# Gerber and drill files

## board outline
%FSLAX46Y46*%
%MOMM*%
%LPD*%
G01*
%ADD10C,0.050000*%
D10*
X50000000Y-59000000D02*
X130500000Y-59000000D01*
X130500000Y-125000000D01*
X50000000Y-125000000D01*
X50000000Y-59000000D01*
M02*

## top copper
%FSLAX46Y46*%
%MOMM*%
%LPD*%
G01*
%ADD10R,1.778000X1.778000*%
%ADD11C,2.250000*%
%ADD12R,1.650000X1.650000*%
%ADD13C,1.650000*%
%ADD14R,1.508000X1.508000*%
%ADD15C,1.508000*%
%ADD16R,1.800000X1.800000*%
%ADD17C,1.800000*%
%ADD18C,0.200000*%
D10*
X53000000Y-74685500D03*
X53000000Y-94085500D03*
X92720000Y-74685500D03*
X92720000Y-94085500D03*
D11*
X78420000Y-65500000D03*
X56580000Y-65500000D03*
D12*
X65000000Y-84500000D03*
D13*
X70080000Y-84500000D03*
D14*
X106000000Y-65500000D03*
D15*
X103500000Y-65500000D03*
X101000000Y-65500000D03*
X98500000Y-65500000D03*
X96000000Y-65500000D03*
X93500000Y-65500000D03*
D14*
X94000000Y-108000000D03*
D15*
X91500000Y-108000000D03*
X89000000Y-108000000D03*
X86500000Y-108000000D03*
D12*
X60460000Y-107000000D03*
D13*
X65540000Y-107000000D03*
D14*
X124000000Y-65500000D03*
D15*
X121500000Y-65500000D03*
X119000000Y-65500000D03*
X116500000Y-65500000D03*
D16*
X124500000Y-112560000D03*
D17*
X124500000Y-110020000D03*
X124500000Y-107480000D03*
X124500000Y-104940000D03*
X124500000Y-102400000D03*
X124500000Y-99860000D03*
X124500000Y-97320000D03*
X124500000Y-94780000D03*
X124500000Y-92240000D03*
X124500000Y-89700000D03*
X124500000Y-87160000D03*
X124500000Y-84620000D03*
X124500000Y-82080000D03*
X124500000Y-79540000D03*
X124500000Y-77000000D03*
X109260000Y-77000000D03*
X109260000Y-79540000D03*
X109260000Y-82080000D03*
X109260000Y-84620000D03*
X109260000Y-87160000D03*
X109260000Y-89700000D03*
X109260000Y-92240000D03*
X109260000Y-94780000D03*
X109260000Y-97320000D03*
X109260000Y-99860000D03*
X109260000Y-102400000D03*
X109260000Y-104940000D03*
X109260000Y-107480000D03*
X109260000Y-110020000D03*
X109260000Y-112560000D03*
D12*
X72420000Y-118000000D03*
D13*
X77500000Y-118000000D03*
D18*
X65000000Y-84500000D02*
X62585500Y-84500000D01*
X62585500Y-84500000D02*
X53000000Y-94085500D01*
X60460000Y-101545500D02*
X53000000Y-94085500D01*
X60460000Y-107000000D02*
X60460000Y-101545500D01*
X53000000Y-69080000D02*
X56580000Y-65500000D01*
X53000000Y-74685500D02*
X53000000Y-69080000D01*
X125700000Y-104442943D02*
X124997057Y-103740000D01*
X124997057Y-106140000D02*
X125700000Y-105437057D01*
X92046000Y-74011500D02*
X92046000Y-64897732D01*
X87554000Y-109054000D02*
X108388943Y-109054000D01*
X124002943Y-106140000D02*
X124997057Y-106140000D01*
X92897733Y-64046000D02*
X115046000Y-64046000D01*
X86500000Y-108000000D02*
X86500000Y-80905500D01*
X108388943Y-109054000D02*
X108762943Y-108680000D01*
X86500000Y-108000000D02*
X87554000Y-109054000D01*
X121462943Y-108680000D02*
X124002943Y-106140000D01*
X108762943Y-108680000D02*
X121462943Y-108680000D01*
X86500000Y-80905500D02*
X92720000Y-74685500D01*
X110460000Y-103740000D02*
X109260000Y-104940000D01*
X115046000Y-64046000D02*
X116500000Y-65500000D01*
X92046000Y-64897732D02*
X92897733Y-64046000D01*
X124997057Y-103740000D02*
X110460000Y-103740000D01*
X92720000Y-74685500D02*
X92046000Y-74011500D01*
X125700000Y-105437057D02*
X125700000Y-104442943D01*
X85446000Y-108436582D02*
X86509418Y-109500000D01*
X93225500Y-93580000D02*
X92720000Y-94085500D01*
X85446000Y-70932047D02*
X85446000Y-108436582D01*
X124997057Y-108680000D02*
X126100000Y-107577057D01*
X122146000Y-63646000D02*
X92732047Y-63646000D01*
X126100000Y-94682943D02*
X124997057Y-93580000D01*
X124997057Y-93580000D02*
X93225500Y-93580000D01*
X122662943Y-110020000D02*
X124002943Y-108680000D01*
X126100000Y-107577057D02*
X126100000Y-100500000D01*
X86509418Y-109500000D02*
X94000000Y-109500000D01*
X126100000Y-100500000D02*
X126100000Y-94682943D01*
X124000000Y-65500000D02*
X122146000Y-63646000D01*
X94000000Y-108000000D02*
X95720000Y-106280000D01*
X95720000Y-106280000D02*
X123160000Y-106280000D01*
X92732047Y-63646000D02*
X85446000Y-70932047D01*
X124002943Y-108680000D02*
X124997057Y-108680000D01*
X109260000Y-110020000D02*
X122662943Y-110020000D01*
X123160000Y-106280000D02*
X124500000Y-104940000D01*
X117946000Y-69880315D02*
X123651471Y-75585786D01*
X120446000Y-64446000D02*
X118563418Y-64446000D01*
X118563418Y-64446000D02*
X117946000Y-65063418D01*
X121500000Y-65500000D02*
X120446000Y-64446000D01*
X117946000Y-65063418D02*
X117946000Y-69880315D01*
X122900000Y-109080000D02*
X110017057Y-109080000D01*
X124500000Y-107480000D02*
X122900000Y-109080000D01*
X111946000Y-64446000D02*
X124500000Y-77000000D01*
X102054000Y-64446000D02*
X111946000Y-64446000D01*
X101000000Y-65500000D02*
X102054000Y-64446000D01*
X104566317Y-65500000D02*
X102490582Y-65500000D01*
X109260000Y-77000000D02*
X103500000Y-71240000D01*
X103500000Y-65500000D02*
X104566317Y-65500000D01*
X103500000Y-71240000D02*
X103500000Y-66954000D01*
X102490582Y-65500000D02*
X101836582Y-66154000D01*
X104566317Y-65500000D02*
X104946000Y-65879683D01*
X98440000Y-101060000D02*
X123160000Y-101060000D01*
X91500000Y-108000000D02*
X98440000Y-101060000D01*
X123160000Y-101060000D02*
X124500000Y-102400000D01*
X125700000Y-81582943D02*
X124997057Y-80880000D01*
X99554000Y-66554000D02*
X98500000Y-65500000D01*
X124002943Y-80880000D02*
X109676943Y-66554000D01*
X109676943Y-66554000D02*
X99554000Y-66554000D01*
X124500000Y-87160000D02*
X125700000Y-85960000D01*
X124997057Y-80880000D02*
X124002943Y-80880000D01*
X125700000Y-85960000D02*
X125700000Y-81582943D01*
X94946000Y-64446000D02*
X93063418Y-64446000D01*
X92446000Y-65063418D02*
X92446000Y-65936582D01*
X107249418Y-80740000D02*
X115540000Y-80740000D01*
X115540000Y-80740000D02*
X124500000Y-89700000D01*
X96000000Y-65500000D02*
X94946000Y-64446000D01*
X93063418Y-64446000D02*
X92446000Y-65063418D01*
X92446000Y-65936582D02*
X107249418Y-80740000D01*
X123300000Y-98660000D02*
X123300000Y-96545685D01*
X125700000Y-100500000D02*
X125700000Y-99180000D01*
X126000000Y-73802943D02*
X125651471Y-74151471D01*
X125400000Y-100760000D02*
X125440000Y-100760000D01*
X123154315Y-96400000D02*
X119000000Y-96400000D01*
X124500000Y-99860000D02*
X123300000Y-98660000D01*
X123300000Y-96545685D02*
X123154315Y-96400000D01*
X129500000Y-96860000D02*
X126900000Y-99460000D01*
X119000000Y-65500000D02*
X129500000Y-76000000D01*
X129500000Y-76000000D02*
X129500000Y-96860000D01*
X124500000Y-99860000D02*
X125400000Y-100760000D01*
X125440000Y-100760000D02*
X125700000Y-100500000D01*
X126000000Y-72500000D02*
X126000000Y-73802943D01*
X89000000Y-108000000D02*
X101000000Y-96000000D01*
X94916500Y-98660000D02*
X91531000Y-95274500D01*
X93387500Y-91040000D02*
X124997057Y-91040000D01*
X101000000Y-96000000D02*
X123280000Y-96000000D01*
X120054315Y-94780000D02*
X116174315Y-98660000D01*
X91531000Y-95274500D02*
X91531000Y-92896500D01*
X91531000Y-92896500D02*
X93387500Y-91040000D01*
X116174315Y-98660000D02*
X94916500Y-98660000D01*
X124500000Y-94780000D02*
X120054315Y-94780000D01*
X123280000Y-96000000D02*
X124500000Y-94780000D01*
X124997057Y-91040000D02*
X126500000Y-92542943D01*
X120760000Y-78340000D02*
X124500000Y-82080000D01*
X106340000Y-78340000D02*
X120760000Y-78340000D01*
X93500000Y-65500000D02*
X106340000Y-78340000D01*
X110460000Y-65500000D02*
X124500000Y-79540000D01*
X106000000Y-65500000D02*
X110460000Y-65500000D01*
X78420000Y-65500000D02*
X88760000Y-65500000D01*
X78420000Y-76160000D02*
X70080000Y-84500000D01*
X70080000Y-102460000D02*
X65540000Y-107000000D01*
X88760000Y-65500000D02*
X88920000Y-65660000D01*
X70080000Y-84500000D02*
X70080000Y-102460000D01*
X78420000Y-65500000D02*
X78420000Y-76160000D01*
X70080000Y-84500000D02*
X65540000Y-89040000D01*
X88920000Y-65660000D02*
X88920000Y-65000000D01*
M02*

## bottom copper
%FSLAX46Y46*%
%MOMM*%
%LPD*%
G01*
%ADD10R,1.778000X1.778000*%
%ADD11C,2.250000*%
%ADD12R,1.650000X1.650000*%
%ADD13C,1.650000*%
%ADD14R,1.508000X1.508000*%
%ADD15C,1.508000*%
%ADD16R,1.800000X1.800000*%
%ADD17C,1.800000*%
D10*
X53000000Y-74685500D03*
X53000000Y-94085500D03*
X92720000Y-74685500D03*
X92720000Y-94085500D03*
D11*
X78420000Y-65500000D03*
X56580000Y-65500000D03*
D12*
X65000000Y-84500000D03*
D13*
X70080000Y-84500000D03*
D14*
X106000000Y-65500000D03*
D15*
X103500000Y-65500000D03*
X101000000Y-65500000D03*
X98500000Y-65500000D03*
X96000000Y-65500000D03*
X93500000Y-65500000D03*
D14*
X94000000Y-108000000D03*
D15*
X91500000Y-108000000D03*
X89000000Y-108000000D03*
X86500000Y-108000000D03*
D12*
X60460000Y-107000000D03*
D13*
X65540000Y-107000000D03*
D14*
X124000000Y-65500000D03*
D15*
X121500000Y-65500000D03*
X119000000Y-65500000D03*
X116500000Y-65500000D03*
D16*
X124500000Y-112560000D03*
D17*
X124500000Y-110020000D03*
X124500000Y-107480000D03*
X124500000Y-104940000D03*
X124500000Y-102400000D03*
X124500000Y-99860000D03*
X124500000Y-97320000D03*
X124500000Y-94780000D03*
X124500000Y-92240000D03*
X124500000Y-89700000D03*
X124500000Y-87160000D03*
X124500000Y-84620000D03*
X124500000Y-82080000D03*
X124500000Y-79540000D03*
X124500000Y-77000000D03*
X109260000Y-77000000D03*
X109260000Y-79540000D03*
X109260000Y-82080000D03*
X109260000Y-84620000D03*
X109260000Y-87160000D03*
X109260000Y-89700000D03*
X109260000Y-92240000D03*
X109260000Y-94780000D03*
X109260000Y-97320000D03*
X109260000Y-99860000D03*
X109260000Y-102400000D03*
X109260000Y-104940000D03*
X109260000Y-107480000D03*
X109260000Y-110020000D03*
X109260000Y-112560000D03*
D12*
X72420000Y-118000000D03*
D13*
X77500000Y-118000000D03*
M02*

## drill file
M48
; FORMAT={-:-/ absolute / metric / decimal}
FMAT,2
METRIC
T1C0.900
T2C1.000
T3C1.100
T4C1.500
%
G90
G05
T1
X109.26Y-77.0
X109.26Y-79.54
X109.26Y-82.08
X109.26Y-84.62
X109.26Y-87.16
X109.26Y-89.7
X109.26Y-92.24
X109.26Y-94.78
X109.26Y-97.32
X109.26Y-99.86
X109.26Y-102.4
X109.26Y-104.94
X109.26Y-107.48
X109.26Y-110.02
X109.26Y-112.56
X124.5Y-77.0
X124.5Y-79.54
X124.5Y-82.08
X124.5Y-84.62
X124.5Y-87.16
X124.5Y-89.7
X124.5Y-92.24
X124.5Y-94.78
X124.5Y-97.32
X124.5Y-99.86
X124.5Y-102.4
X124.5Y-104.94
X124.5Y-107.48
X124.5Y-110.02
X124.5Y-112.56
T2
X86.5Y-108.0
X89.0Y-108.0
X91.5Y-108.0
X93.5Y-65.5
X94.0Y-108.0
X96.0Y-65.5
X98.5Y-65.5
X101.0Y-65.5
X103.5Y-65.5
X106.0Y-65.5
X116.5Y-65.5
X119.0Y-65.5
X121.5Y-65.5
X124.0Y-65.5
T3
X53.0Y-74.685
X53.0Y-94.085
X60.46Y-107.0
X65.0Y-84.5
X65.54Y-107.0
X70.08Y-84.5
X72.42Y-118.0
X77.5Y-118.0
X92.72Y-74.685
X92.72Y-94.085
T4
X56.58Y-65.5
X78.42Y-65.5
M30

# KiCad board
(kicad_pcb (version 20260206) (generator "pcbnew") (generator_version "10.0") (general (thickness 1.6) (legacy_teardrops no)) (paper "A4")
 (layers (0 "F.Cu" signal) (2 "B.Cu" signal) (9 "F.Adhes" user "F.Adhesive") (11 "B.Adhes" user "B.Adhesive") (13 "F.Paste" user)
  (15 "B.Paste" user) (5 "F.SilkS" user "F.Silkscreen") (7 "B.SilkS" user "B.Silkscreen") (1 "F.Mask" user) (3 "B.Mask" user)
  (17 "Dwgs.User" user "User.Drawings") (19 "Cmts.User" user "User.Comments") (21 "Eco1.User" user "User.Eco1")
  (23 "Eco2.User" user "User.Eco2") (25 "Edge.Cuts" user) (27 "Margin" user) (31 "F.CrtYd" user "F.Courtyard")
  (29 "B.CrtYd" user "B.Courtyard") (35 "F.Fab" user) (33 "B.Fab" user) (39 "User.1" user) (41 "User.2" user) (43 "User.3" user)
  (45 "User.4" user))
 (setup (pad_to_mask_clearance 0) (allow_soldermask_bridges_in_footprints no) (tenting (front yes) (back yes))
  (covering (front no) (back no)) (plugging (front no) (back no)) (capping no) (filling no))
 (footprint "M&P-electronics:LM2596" (layer "F.Cu") (at 53 74.6855)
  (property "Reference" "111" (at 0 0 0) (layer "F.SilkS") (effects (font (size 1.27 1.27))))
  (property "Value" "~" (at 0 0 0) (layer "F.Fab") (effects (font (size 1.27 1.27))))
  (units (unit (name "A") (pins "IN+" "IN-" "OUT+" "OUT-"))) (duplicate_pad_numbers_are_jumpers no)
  (pad "IN+" thru_hole rect (at 0 0) (size 1.778 1.778) (drill 1.1) (layers "*.Cu" "*.Mask") (remove_unused_layers no)
   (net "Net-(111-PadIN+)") (solder_mask_margin 0.1016) (thermal_bridge_angle 0))
  (pad "IN-" thru_hole rect (at 0 19.4) (size 1.778 1.778) (drill 1.1) (layers "*.Cu" "*.Mask") (remove_unused_layers no)
   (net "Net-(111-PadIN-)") (solder_mask_margin 0.1016) (thermal_bridge_angle 0))
  (pad "OUT+" thru_hole rect (at 39.72 0) (size 1.778 1.778) (drill 1.1) (layers "*.Cu" "*.Mask") (remove_unused_layers no) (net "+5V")
   (solder_mask_margin 0.1016) (thermal_bridge_angle 0))
  (pad "OUT-" thru_hole rect (at 39.72 19.4) (size 1.778 1.778) (drill 1.1) (layers "*.Cu" "*.Mask") (remove_unused_layers no) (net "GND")
   (solder_mask_margin 0.1016) (thermal_bridge_angle 0)))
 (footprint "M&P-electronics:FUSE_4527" (layer "F.Cu") (at 67.5 65.5 180)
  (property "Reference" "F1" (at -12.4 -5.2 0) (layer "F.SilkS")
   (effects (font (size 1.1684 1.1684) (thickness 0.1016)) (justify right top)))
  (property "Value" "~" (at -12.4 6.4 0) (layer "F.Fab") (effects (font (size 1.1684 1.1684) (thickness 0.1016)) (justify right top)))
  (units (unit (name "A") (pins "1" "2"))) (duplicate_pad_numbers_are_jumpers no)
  (pad "1" thru_hole circle (at -10.92 0 180) (size 2.25 2.25) (drill 1.5) (layers "*.Cu" "*.Mask") (remove_unused_layers no)
   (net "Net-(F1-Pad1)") (solder_mask_margin 0.1016) (thermal_bridge_angle 0))
  (pad "2" thru_hole circle (at 10.92 0 180) (size 2.25 2.25) (drill 1.5) (layers "*.Cu" "*.Mask") (remove_unused_layers no)
   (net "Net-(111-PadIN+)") (solder_mask_margin 0.1016) (thermal_bridge_angle 0)))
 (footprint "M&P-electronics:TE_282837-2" (layer "F.Cu") (at 67.54 84.5)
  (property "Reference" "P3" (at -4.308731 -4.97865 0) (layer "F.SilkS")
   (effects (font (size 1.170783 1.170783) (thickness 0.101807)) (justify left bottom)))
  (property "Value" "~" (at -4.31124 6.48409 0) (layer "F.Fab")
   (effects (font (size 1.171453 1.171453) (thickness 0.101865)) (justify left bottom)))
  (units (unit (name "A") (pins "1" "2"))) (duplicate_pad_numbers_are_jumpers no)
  (pad "1" thru_hole rect (at -2.54 0) (size 1.65 1.65) (drill 1.1) (layers "*.Cu" "*.Mask") (remove_unused_layers no)
   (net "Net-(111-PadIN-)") (solder_mask_margin 0.1016) (thermal_bridge_angle 0))
  (pad "2" thru_hole circle (at 2.54 0) (size 1.65 1.65) (drill 1.1) (layers "*.Cu" "*.Mask") (remove_unused_layers no)
   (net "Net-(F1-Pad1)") (solder_mask_margin 0.1016) (thermal_bridge_angle 0)))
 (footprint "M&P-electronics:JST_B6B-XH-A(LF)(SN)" (layer "F.Cu") (at 99.75 64.975)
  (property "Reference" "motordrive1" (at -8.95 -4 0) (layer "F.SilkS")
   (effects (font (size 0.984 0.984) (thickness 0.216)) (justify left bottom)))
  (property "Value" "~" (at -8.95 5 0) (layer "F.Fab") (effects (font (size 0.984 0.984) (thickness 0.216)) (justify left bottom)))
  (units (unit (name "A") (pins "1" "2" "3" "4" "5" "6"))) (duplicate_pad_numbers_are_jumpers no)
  (pad "1" thru_hole rect (at 6.25 0.525) (size 1.508 1.508) (drill 1) (layers "*.Cu" "*.Mask") (remove_unused_layers no) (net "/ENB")
   (solder_mask_margin 0.1016) (thermal_bridge_angle 0))
  (pad "2" thru_hole circle (at 3.75 0.525) (size 1.508 1.508) (drill 1) (layers "*.Cu" "*.Mask") (remove_unused_layers no) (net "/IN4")
   (solder_mask_margin 0.1016) (thermal_bridge_angle 0))
  (pad "3" thru_hole circle (at 1.25 0.525) (size 1.508 1.508) (drill 1) (layers "*.Cu" "*.Mask") (remove_unused_layers no) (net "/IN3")
   (solder_mask_margin 0.1016) (thermal_bridge_angle 0))
  (pad "4" thru_hole circle (at -1.25 0.525) (size 1.508 1.508) (drill 1) (layers "*.Cu" "*.Mask") (remove_unused_layers no) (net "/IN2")
   (solder_mask_margin 0.1016) (thermal_bridge_angle 0))
  (pad "5" thru_hole circle (at -3.75 0.525) (size 1.508 1.508) (drill 1) (layers "*.Cu" "*.Mask") (remove_unused_layers no) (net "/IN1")
   (solder_mask_margin 0.1016) (thermal_bridge_angle 0))
  (pad "6" thru_hole circle (at -6.25 0.525) (size 1.508 1.508) (drill 1) (layers "*.Cu" "*.Mask") (remove_unused_layers no) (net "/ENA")
   (solder_mask_margin 0.1016) (thermal_bridge_angle 0)))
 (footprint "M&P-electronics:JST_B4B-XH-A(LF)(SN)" (layer "F.Cu") (at 90.25 107.475)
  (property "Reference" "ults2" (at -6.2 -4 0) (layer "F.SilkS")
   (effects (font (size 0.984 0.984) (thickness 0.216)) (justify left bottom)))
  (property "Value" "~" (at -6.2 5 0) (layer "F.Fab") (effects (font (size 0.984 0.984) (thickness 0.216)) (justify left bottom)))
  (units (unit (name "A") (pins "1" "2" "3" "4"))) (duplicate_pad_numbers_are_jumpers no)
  (pad "1" thru_hole rect (at 3.75 0.525) (size 1.508 1.508) (drill 1) (layers "*.Cu" "*.Mask") (remove_unused_layers no) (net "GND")
   (solder_mask_margin 0.1016) (thermal_bridge_angle 0))
  (pad "2" thru_hole circle (at 1.25 0.525) (size 1.508 1.508) (drill 1) (layers "*.Cu" "*.Mask") (remove_unused_layers no) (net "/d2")
   (solder_mask_margin 0.1016) (thermal_bridge_angle 0))
  (pad "3" thru_hole circle (at -1.25 0.525) (size 1.508 1.508) (drill 1) (layers "*.Cu" "*.Mask") (remove_unused_layers no) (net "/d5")
   (solder_mask_margin 0.1016) (thermal_bridge_angle 0))
  (pad "4" thru_hole circle (at -3.75 0.525) (size 1.508 1.508) (drill 1) (layers "*.Cu" "*.Mask") (remove_unused_layers no) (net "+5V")
   (solder_mask_margin 0.1016) (thermal_bridge_angle 0)))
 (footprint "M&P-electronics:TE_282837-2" (layer "F.Cu") (at 63 107)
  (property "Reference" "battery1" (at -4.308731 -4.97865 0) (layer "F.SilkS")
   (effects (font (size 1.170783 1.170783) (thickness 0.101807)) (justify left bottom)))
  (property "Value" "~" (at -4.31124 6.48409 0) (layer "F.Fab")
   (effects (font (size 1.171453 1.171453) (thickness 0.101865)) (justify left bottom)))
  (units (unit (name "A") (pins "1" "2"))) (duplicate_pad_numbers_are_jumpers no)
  (pad "1" thru_hole rect (at -2.54 0) (size 1.65 1.65) (drill 1.1) (layers "*.Cu" "*.Mask") (remove_unused_layers no)
   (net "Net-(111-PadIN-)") (solder_mask_margin 0.1016) (thermal_bridge_angle 0))
  (pad "2" thru_hole circle (at 2.54 0) (size 1.65 1.65) (drill 1.1) (layers "*.Cu" "*.Mask") (remove_unused_layers no)
   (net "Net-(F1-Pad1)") (solder_mask_margin 0.1016) (thermal_bridge_angle 0)))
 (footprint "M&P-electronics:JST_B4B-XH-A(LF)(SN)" (layer "F.Cu") (at 120.25 64.975)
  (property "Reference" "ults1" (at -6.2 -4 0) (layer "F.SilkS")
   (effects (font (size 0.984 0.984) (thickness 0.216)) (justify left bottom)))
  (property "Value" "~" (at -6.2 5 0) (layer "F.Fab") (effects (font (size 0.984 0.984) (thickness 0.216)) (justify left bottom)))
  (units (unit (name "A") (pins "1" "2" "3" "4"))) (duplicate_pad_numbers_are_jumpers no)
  (pad "1" thru_hole rect (at 3.75 0.525) (size 1.508 1.508) (drill 1) (layers "*.Cu" "*.Mask") (remove_unused_layers no) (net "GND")
   (solder_mask_margin 0.1016) (thermal_bridge_angle 0))
  (pad "2" thru_hole circle (at 1.25 0.525) (size 1.508 1.508) (drill 1) (layers "*.Cu" "*.Mask") (remove_unused_layers no) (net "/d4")
   (solder_mask_margin 0.1016) (thermal_bridge_angle 0))
  (pad "3" thru_hole circle (at -1.25 0.525) (size 1.508 1.508) (drill 1) (layers "*.Cu" "*.Mask") (remove_unused_layers no) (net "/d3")
   (solder_mask_margin 0.1016) (thermal_bridge_angle 0))
  (pad "4" thru_hole circle (at -3.75 0.525) (size 1.508 1.508) (drill 1) (layers "*.Cu" "*.Mask") (remove_unused_layers no) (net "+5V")
   (solder_mask_margin 0.1016) (thermal_bridge_angle 0)))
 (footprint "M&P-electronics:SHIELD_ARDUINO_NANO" (layer "F.Cu") (at 116.88 94.78 180)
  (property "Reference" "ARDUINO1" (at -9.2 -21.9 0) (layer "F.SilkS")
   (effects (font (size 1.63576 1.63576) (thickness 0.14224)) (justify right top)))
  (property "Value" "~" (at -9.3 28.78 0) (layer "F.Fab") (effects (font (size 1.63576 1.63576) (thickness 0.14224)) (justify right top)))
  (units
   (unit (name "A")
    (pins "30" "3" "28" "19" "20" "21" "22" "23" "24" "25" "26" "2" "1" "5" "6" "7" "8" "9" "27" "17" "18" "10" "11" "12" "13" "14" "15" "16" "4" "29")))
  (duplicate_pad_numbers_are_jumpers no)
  (pad "1" thru_hole rect (at -7.62 -17.78 90) (size 1.8 1.8) (drill 0.9) (layers "*.Cu" "*.Mask") (remove_unused_layers no)
   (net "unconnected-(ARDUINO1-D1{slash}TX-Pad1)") (solder_mask_margin 0.1016) (thermal_bridge_angle 0))
  (pad "2" thru_hole circle (at -7.62 -15.24 90) (size 1.8 1.8) (drill 0.9) (layers "*.Cu" "*.Mask") (remove_unused_layers no)
   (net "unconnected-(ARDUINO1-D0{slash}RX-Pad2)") (solder_mask_margin 0.1016) (thermal_bridge_angle 0))
  (pad "3" thru_hole circle (at -7.62 -12.7 90) (size 1.8 1.8) (drill 0.9) (layers "*.Cu" "*.Mask") (remove_unused_layers no)
   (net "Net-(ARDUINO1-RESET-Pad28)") (solder_mask_margin 0.1016) (thermal_bridge_angle 0))
  (pad "4" thru_hole circle (at -7.62 -10.16 90) (size 1.8 1.8) (drill 0.9) (layers "*.Cu" "*.Mask") (remove_unused_layers no) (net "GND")
   (solder_mask_margin 0.1016) (thermal_bridge_angle 0))
  (pad "5" thru_hole circle (at -7.62 -7.62 90) (size 1.8 1.8) (drill 0.9) (layers "*.Cu" "*.Mask") (remove_unused_layers no) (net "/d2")
   (solder_mask_margin 0.1016) (thermal_bridge_angle 0))
  (pad "6" thru_hole circle (at -7.62 -5.08 90) (size 1.8 1.8) (drill 0.9) (layers "*.Cu" "*.Mask") (remove_unused_layers no) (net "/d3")
   (solder_mask_margin 0.1016) (thermal_bridge_angle 0))
  (pad "7" thru_hole circle (at -7.62 -2.54 90) (size 1.8 1.8) (drill 0.9) (layers "*.Cu" "*.Mask") (remove_unused_layers no) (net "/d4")
   (solder_mask_margin 0.1016) (thermal_bridge_angle 0))
  (pad "8" thru_hole circle (at -7.62 0 90) (size 1.8 1.8) (drill 0.9) (layers "*.Cu" "*.Mask") (remove_unused_layers no) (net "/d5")
   (solder_mask_margin 0.1016) (thermal_bridge_angle 0))
  (pad "9" thru_hole circle (at -7.62 2.54 90) (size 1.8 1.8) (drill 0.9) (layers "*.Cu" "*.Mask") (remove_unused_layers no) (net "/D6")
   (solder_mask_margin 0.1016) (thermal_bridge_angle 0))
  (pad "10" thru_hole circle (at -7.62 5.08 90) (size 1.8 1.8) (drill 0.9) (layers "*.Cu" "*.Mask") (remove_unused_layers no) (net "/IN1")
   (solder_mask_margin 0.1016) (thermal_bridge_angle 0))
  (pad "11" thru_hole circle (at -7.62 7.62 90) (size 1.8 1.8) (drill 0.9) (layers "*.Cu" "*.Mask") (remove_unused_layers no) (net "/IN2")
   (solder_mask_margin 0.1016) (thermal_bridge_angle 0))
  (pad "12" thru_hole circle (at -7.62 10.16 90) (size 1.8 1.8) (drill 0.9) (layers "*.Cu" "*.Mask") (remove_unused_layers no)
   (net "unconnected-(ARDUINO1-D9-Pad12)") (solder_mask_margin 0.1016) (thermal_bridge_angle 0))
  (pad "13" thru_hole circle (at -7.62 12.7 90) (size 1.8 1.8) (drill 0.9) (layers "*.Cu" "*.Mask") (remove_unused_layers no) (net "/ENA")
   (solder_mask_margin 0.1016) (thermal_bridge_angle 0))
  (pad "14" thru_hole circle (at -7.62 15.24 90) (size 1.8 1.8) (drill 0.9) (layers "*.Cu" "*.Mask") (remove_unused_layers no) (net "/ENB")
   (solder_mask_margin 0.1016) (thermal_bridge_angle 0))
  (pad "15" thru_hole circle (at -7.62 17.78 90) (size 1.8 1.8) (drill 0.9) (layers "*.Cu" "*.Mask") (remove_unused_layers no) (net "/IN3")
   (solder_mask_margin 0.1016) (thermal_bridge_angle 0))
  (pad "16" thru_hole circle (at 7.62 17.78 270) (size 1.8 1.8) (drill 0.9) (layers "*.Cu" "*.Mask") (remove_unused_layers no) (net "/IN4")
   (solder_mask_margin 0.1016) (thermal_bridge_angle 0))
  (pad "17" thru_hole circle (at 7.62 15.24 270) (size 1.8 1.8) (drill 0.9) (layers "*.Cu" "*.Mask") (remove_unused_layers no)
   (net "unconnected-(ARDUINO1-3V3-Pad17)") (solder_mask_margin 0.1016) (thermal_bridge_angle 0))
  (pad "18" thru_hole circle (at 7.62 12.7 270) (size 1.8 1.8) (drill 0.9) (layers "*.Cu" "*.Mask") (remove_unused_layers no)
   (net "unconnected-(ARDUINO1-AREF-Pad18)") (solder_mask_margin 0.1016) (thermal_bridge_angle 0))
  (pad "19" thru_hole circle (at 7.62 10.16 270) (size 1.8 1.8) (drill 0.9) (layers "*.Cu" "*.Mask") (remove_unused_layers no) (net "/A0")
   (solder_mask_margin 0.1016) (thermal_bridge_angle 0))
  (pad "20" thru_hole circle (at 7.62 7.62 270) (size 1.8 1.8) (drill 0.9) (layers "*.Cu" "*.Mask") (remove_unused_layers no)
   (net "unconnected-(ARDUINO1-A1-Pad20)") (solder_mask_margin 0.1016) (thermal_bridge_angle 0))
  (pad "21" thru_hole circle (at 7.62 5.08 270) (size 1.8 1.8) (drill 0.9) (layers "*.Cu" "*.Mask") (remove_unused_layers no) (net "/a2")
   (solder_mask_margin 0.1016) (thermal_bridge_angle 0))
  (pad "22" thru_hole circle (at 7.62 2.54 270) (size 1.8 1.8) (drill 0.9) (layers "*.Cu" "*.Mask") (remove_unused_layers no) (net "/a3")
   (solder_mask_margin 0.1016) (thermal_bridge_angle 0))
  (pad "23" thru_hole circle (at 7.62 0 270) (size 1.8 1.8) (drill 0.9) (layers "*.Cu" "*.Mask") (remove_unused_layers no)
   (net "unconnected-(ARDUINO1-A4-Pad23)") (solder_mask_margin 0.1016) (thermal_bridge_angle 0))
  (pad "24" thru_hole circle (at 7.62 -2.54 270) (size 1.8 1.8) (drill 0.9) (layers "*.Cu" "*.Mask") (remove_unused_layers no)
   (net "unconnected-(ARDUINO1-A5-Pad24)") (solder_mask_margin 0.1016) (thermal_bridge_angle 0))
  (pad "25" thru_hole circle (at 7.62 -5.08 270) (size 1.8 1.8) (drill 0.9) (layers "*.Cu" "*.Mask") (remove_unused_layers no)
   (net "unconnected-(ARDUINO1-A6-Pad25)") (solder_mask_margin 0.1016) (thermal_bridge_angle 0))
  (pad "26" thru_hole circle (at 7.62 -7.62 270) (size 1.8 1.8) (drill 0.9) (layers "*.Cu" "*.Mask") (remove_unused_layers no)
   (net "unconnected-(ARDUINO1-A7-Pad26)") (solder_mask_margin 0.1016) (thermal_bridge_angle 0))
  (pad "27" thru_hole circle (at 7.62 -10.16 270) (size 1.8 1.8) (drill 0.9) (layers "*.Cu" "*.Mask") (remove_unused_layers no) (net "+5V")
   (solder_mask_margin 0.1016) (thermal_bridge_angle 0))
  (pad "28" thru_hole circle (at 7.62 -12.7 270) (size 1.8 1.8) (drill 0.9) (layers "*.Cu" "*.Mask") (remove_unused_layers no)
   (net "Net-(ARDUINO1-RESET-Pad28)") (solder_mask_margin 0.1016) (thermal_bridge_angle 0))
  (pad "29" thru_hole circle (at 7.62 -15.24 270) (size 1.8 1.8) (drill 0.9) (layers "*.Cu" "*.Mask") (remove_unused_layers no) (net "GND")
   (solder_mask_margin 0.1016) (thermal_bridge_angle 0))
  (pad "30" thru_hole circle (at 7.62 -17.78 270) (size 1.8 1.8) (drill 0.9) (layers "*.Cu" "*.Mask") (remove_unused_layers no)
   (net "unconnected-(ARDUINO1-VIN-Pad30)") (solder_mask_margin 0.1016) (thermal_bridge_angle 0)))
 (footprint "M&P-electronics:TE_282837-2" (layer "F.Cu") (at 74.96 118)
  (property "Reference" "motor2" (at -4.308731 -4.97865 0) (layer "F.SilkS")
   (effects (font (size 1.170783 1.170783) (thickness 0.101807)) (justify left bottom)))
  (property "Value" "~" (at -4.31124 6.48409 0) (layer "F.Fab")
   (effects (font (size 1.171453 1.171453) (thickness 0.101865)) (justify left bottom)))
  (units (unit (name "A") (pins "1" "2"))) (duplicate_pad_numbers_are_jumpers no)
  (pad "1" thru_hole rect (at -2.54 0) (size 1.65 1.65) (drill 1.1) (layers "*.Cu" "*.Mask") (remove_unused_layers no)
   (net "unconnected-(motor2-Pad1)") (solder_mask_margin 0.1016) (thermal_bridge_angle 0))
  (pad "2" thru_hole circle (at 2.54 0) (size 1.65 1.65) (drill 1.1) (layers "*.Cu" "*.Mask") (remove_unused_layers no)
   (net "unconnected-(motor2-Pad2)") (solder_mask_margin 0.1016) (thermal_bridge_angle 0)))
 (gr_rect (start 50 59) (end 130.5 125) (stroke (width 0.05) (type default)) (fill no) (layer "Edge.Cuts"))
 (segment (start 65 84.5) (end 62.5855 84.5) (width 0.2) (layer "F.Cu") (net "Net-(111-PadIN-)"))
 (segment (start 62.5855 84.5) (end 53 94.0855) (width 0.2) (layer "F.Cu") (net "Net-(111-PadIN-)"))
 (segment (start 60.46 101.5455) (end 53 94.0855) (width 0.2) (layer "F.Cu") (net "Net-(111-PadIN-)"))
 (segment (start 60.46 107) (end 60.46 101.5455) (width 0.2) (layer "F.Cu") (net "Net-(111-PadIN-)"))
 (segment (start 53 69.08) (end 56.58 65.5) (width 0.2) (layer "F.Cu") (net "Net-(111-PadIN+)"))
 (segment (start 53 74.6855) (end 53 69.08) (width 0.2) (layer "F.Cu") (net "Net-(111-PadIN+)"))
 (segment (start 125.7 104.442943) (end 124.997057 103.74) (width 0.2) (layer "F.Cu") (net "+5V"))
 (segment (start 124.997057 106.14) (end 125.7 105.437057) (width 0.2) (layer "F.Cu") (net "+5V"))
 (segment (start 92.046 74.0115) (end 92.046 64.897732) (width 0.2) (layer "F.Cu") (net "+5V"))
 (segment (start 87.554 109.054) (end 108.388943 109.054) (width 0.2) (layer "F.Cu") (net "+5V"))
 (segment (start 124.002943 106.14) (end 124.997057 106.14) (width 0.2) (layer "F.Cu") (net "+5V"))
 (segment (start 92.897733 64.046) (end 115.046 64.046) (width 0.2) (layer "F.Cu") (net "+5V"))
 (segment (start 86.5 108) (end 86.5 80.9055) (width 0.2) (layer "F.Cu") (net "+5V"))
 (segment (start 108.388943 109.054) (end 108.762943 108.68) (width 0.2) (layer "F.Cu") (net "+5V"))
 (segment (start 86.5 108) (end 87.554 109.054) (width 0.2) (layer "F.Cu") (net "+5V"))
 (segment (start 121.462943 108.68) (end 124.002943 106.14) (width 0.2) (layer "F.Cu") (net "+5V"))
 (segment (start 108.762943 108.68) (end 121.462943 108.68) (width 0.2) (layer "F.Cu") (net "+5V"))
 (segment (start 86.5 80.9055) (end 92.72 74.6855) (width 0.2) (layer "F.Cu") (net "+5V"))
 (segment (start 110.46 103.74) (end 109.26 104.94) (width 0.2) (layer "F.Cu") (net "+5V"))
 (segment (start 115.046 64.046) (end 116.5 65.5) (width 0.2) (layer "F.Cu") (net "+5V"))
 (segment (start 92.046 64.897732) (end 92.897733 64.046) (width 0.2) (layer "F.Cu") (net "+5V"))
 (segment (start 124.997057 103.74) (end 110.46 103.74) (width 0.2) (layer "F.Cu") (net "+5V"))
 (segment (start 92.72 74.6855) (end 92.046 74.0115) (width 0.2) (layer "F.Cu") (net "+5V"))
 (segment (start 125.7 105.437057) (end 125.7 104.442943) (width 0.2) (layer "F.Cu") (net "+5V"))
 (segment (start 85.446 108.436582) (end 86.509418 109.5) (width 0.2) (layer "F.Cu") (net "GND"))
 (segment (start 93.2255 93.58) (end 92.72 94.0855) (width 0.2) (layer "F.Cu") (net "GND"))
 (segment (start 85.446 70.932047) (end 85.446 108.436582) (width 0.2) (layer "F.Cu") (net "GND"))
 (segment (start 124.997057 108.68) (end 126.1 107.577057) (width 0.2) (layer "F.Cu") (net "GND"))
 (segment (start 122.146 63.646) (end 92.732047 63.646) (width 0.2) (layer "F.Cu") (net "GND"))
 (segment (start 126.1 94.682943) (end 124.997057 93.58) (width 0.2) (layer "F.Cu") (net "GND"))
 (segment (start 124.997057 93.58) (end 93.2255 93.58) (width 0.2) (layer "F.Cu") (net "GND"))
 (segment (start 122.662943 110.02) (end 124.002943 108.68) (width 0.2) (layer "F.Cu") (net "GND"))
 (segment (start 126.1 107.577057) (end 126.1 100.5) (width 0.2) (layer "F.Cu") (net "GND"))
 (segment (start 86.509418 109.5) (end 94 109.5) (width 0.2) (layer "F.Cu") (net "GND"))
 (segment (start 126.1 100.5) (end 126.1 94.682943) (width 0.2) (layer "F.Cu") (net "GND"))
 (segment (start 124 65.5) (end 122.146 63.646) (width 0.2) (layer "F.Cu") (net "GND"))
 (segment (start 94 108) (end 95.72 106.28) (width 0.2) (layer "F.Cu") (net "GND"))
 (segment (start 95.72 106.28) (end 123.16 106.28) (width 0.2) (layer "F.Cu") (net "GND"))
 (segment (start 92.732047 63.646) (end 85.446 70.932047) (width 0.2) (layer "F.Cu") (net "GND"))
 (segment (start 124.002943 108.68) (end 124.997057 108.68) (width 0.2) (layer "F.Cu") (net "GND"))
 (segment (start 109.26 110.02) (end 122.662943 110.02) (width 0.2) (layer "F.Cu") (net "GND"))
 (segment (start 123.16 106.28) (end 124.5 104.94) (width 0.2) (layer "F.Cu") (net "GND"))
 (segment (start 117.946 69.880315) (end 123.651471 75.585786) (width 0.2) (layer "F.Cu") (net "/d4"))
 (segment (start 120.446 64.446) (end 118.563418 64.446) (width 0.2) (layer "F.Cu") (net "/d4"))
 (segment (start 118.563418 64.446) (end 117.946 65.063418) (width 0.2) (layer "F.Cu") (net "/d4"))
 (segment (start 121.5 65.5) (end 120.446 64.446) (width 0.2) (layer "F.Cu") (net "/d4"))
 (segment (start 117.946 65.063418) (end 117.946 69.880315) (width 0.2) (layer "F.Cu") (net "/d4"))
 (segment (start 122.9 109.08) (end 110.017057 109.08) (width 0.2) (layer "F.Cu") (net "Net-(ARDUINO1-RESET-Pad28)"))
 (segment (start 124.5 107.48) (end 122.9 109.08) (width 0.2) (layer "F.Cu") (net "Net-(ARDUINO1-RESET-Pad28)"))
 (segment (start 111.946 64.446) (end 124.5 77) (width 0.2) (layer "F.Cu") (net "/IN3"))
 (segment (start 102.054 64.446) (end 111.946 64.446) (width 0.2) (layer "F.Cu") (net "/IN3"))
 (segment (start 101 65.5) (end 102.054 64.446) (width 0.2) (layer "F.Cu") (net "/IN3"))
 (segment (start 104.566317 65.5) (end 102.490582 65.5) (width 0.2) (layer "F.Cu") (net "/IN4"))
 (segment (start 109.26 77) (end 103.5 71.24) (width 0.2) (layer "F.Cu") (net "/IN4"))
 (segment (start 103.5 65.5) (end 104.566317 65.5) (width 0.2) (layer "F.Cu") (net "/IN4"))
 (segment (start 103.5 71.24) (end 103.5 66.954) (width 0.2) (layer "F.Cu") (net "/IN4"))
 (segment (start 102.490582 65.5) (end 101.836582 66.154) (width 0.2) (layer "F.Cu") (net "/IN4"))
 (segment (start 104.566317 65.5) (end 104.946 65.879683) (width 0.2) (layer "F.Cu") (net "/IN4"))
 (segment (start 98.44 101.06) (end 123.16 101.06) (width 0.2) (layer "F.Cu") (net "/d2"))
 (segment (start 91.5 108) (end 98.44 101.06) (width 0.2) (layer "F.Cu") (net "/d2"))
 (segment (start 123.16 101.06) (end 124.5 102.4) (width 0.2) (layer "F.Cu") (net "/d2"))
 (segment (start 125.7 81.582943) (end 124.997057 80.88) (width 0.2) (layer "F.Cu") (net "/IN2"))
 (segment (start 99.554 66.554) (end 98.5 65.5) (width 0.2) (layer "F.Cu") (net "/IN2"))
 (segment (start 124.002943 80.88) (end 109.676943 66.554) (width 0.2) (layer "F.Cu") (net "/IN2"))
 (segment (start 109.676943 66.554) (end 99.554 66.554) (width 0.2) (layer "F.Cu") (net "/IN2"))
 (segment (start 124.5 87.16) (end 125.7 85.96) (width 0.2) (layer "F.Cu") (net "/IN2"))
 (segment (start 124.997057 80.88) (end 124.002943 80.88) (width 0.2) (layer "F.Cu") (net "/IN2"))
 (segment (start 125.7 85.96) (end 125.7 81.582943) (width 0.2) (layer "F.Cu") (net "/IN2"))
 (segment (start 94.946 64.446) (end 93.063418 64.446) (width 0.2) (layer "F.Cu") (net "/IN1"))
 (segment (start 92.446 65.063418) (end 92.446 65.936582) (width 0.2) (layer "F.Cu") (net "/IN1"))
 (segment (start 107.249418 80.74) (end 115.54 80.74) (width 0.2) (layer "F.Cu") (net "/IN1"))
 (segment (start 115.54 80.74) (end 124.5 89.7) (width 0.2) (layer "F.Cu") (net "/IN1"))
 (segment (start 96 65.5) (end 94.946 64.446) (width 0.2) (layer "F.Cu") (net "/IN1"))
 (segment (start 93.063418 64.446) (end 92.446 65.063418) (width 0.2) (layer "F.Cu") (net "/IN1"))
 (segment (start 92.446 65.936582) (end 107.249418 80.74) (width 0.2) (layer "F.Cu") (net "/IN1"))
 (segment (start 123.3 98.66) (end 123.3 96.545685) (width 0.2) (layer "F.Cu") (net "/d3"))
 (segment (start 125.7 100.5) (end 125.7 99.18) (width 0.2) (layer "F.Cu") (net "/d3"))
 (segment (start 126 73.802943) (end 125.651471 74.151471) (width 0.2) (layer "F.Cu") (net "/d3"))
 (segment (start 125.4 100.76) (end 125.44 100.76) (width 0.2) (layer "F.Cu") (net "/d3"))
 (segment (start 123.154315 96.4) (end 119 96.4) (width 0.2) (layer "F.Cu") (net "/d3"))
 (segment (start 124.5 99.86) (end 123.3 98.66) (width 0.2) (layer "F.Cu") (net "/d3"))
 (segment (start 123.3 96.545685) (end 123.154315 96.4) (width 0.2) (layer "F.Cu") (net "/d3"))
 (segment (start 129.5 96.86) (end 126.9 99.46) (width 0.2) (layer "F.Cu") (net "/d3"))
 (segment (start 119 65.5) (end 129.5 76) (width 0.2) (layer "F.Cu") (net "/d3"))
 (segment (start 129.5 76) (end 129.5 96.86) (width 0.2) (layer "F.Cu") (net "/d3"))
 (segment (start 124.5 99.86) (end 125.4 100.76) (width 0.2) (layer "F.Cu") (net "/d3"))
 (segment (start 125.44 100.76) (end 125.7 100.5) (width 0.2) (layer "F.Cu") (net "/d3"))
 (segment (start 126 72.5) (end 126 73.802943) (width 0.2) (layer "F.Cu") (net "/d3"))
 (segment (start 89 108) (end 101 96) (width 0.2) (layer "F.Cu") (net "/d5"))
 (segment (start 94.9165 98.66) (end 91.531 95.2745) (width 0.2) (layer "F.Cu") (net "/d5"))
 (segment (start 93.3875 91.04) (end 124.997057 91.04) (width 0.2) (layer "F.Cu") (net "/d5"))
 (segment (start 101 96) (end 123.28 96) (width 0.2) (layer "F.Cu") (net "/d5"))
 (segment (start 120.054315 94.78) (end 116.174315 98.66) (width 0.2) (layer "F.Cu") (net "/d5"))
 (segment (start 91.531 95.2745) (end 91.531 92.8965) (width 0.2) (layer "F.Cu") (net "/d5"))
 (segment (start 91.531 92.8965) (end 93.3875 91.04) (width 0.2) (layer "F.Cu") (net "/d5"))
 (segment (start 116.174315 98.66) (end 94.9165 98.66) (width 0.2) (layer "F.Cu") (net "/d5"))
 (segment (start 124.5 94.78) (end 120.054315 94.78) (width 0.2) (layer "F.Cu") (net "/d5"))
 (segment (start 123.28 96) (end 124.5 94.78) (width 0.2) (layer "F.Cu") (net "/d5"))
 (segment (start 124.997057 91.04) (end 126.5 92.542943) (width 0.2) (layer "F.Cu") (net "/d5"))
 (segment (start 120.76 78.34) (end 124.5 82.08) (width 0.2) (layer "F.Cu") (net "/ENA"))
 (segment (start 106.34 78.34) (end 120.76 78.34) (width 0.2) (layer "F.Cu") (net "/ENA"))
 (segment (start 93.5 65.5) (end 106.34 78.34) (width 0.2) (layer "F.Cu") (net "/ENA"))
 (segment (start 110.46 65.5) (end 124.5 79.54) (width 0.2) (layer "F.Cu") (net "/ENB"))
 (segment (start 106 65.5) (end 110.46 65.5) (width 0.2) (layer "F.Cu") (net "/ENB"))
 (segment (start 78.42 65.5) (end 88.76 65.5) (width 0.2) (layer "F.Cu") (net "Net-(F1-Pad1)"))
 (segment (start 78.42 76.16) (end 70.08 84.5) (width 0.2) (layer "F.Cu") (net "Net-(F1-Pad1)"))
 (segment (start 70.08 102.46) (end 65.54 107) (width 0.2) (layer "F.Cu") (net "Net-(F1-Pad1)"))
 (segment (start 88.76 65.5) (end 88.92 65.66) (width 0.2) (layer "F.Cu") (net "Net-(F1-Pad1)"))
 (segment (start 70.08 84.5) (end 70.08 102.46) (width 0.2) (layer "F.Cu") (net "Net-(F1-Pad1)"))
 (segment (start 78.42 65.5) (end 78.42 76.16) (width 0.2) (layer "F.Cu") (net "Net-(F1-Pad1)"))
 (segment (start 70.08 84.5) (end 65.54 89.04) (width 0.2) (layer "F.Cu") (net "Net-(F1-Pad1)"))
 (segment (start 88.92 65.66) (end 88.92 65) (width 0.2) (layer "F.Cu") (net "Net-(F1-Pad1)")))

